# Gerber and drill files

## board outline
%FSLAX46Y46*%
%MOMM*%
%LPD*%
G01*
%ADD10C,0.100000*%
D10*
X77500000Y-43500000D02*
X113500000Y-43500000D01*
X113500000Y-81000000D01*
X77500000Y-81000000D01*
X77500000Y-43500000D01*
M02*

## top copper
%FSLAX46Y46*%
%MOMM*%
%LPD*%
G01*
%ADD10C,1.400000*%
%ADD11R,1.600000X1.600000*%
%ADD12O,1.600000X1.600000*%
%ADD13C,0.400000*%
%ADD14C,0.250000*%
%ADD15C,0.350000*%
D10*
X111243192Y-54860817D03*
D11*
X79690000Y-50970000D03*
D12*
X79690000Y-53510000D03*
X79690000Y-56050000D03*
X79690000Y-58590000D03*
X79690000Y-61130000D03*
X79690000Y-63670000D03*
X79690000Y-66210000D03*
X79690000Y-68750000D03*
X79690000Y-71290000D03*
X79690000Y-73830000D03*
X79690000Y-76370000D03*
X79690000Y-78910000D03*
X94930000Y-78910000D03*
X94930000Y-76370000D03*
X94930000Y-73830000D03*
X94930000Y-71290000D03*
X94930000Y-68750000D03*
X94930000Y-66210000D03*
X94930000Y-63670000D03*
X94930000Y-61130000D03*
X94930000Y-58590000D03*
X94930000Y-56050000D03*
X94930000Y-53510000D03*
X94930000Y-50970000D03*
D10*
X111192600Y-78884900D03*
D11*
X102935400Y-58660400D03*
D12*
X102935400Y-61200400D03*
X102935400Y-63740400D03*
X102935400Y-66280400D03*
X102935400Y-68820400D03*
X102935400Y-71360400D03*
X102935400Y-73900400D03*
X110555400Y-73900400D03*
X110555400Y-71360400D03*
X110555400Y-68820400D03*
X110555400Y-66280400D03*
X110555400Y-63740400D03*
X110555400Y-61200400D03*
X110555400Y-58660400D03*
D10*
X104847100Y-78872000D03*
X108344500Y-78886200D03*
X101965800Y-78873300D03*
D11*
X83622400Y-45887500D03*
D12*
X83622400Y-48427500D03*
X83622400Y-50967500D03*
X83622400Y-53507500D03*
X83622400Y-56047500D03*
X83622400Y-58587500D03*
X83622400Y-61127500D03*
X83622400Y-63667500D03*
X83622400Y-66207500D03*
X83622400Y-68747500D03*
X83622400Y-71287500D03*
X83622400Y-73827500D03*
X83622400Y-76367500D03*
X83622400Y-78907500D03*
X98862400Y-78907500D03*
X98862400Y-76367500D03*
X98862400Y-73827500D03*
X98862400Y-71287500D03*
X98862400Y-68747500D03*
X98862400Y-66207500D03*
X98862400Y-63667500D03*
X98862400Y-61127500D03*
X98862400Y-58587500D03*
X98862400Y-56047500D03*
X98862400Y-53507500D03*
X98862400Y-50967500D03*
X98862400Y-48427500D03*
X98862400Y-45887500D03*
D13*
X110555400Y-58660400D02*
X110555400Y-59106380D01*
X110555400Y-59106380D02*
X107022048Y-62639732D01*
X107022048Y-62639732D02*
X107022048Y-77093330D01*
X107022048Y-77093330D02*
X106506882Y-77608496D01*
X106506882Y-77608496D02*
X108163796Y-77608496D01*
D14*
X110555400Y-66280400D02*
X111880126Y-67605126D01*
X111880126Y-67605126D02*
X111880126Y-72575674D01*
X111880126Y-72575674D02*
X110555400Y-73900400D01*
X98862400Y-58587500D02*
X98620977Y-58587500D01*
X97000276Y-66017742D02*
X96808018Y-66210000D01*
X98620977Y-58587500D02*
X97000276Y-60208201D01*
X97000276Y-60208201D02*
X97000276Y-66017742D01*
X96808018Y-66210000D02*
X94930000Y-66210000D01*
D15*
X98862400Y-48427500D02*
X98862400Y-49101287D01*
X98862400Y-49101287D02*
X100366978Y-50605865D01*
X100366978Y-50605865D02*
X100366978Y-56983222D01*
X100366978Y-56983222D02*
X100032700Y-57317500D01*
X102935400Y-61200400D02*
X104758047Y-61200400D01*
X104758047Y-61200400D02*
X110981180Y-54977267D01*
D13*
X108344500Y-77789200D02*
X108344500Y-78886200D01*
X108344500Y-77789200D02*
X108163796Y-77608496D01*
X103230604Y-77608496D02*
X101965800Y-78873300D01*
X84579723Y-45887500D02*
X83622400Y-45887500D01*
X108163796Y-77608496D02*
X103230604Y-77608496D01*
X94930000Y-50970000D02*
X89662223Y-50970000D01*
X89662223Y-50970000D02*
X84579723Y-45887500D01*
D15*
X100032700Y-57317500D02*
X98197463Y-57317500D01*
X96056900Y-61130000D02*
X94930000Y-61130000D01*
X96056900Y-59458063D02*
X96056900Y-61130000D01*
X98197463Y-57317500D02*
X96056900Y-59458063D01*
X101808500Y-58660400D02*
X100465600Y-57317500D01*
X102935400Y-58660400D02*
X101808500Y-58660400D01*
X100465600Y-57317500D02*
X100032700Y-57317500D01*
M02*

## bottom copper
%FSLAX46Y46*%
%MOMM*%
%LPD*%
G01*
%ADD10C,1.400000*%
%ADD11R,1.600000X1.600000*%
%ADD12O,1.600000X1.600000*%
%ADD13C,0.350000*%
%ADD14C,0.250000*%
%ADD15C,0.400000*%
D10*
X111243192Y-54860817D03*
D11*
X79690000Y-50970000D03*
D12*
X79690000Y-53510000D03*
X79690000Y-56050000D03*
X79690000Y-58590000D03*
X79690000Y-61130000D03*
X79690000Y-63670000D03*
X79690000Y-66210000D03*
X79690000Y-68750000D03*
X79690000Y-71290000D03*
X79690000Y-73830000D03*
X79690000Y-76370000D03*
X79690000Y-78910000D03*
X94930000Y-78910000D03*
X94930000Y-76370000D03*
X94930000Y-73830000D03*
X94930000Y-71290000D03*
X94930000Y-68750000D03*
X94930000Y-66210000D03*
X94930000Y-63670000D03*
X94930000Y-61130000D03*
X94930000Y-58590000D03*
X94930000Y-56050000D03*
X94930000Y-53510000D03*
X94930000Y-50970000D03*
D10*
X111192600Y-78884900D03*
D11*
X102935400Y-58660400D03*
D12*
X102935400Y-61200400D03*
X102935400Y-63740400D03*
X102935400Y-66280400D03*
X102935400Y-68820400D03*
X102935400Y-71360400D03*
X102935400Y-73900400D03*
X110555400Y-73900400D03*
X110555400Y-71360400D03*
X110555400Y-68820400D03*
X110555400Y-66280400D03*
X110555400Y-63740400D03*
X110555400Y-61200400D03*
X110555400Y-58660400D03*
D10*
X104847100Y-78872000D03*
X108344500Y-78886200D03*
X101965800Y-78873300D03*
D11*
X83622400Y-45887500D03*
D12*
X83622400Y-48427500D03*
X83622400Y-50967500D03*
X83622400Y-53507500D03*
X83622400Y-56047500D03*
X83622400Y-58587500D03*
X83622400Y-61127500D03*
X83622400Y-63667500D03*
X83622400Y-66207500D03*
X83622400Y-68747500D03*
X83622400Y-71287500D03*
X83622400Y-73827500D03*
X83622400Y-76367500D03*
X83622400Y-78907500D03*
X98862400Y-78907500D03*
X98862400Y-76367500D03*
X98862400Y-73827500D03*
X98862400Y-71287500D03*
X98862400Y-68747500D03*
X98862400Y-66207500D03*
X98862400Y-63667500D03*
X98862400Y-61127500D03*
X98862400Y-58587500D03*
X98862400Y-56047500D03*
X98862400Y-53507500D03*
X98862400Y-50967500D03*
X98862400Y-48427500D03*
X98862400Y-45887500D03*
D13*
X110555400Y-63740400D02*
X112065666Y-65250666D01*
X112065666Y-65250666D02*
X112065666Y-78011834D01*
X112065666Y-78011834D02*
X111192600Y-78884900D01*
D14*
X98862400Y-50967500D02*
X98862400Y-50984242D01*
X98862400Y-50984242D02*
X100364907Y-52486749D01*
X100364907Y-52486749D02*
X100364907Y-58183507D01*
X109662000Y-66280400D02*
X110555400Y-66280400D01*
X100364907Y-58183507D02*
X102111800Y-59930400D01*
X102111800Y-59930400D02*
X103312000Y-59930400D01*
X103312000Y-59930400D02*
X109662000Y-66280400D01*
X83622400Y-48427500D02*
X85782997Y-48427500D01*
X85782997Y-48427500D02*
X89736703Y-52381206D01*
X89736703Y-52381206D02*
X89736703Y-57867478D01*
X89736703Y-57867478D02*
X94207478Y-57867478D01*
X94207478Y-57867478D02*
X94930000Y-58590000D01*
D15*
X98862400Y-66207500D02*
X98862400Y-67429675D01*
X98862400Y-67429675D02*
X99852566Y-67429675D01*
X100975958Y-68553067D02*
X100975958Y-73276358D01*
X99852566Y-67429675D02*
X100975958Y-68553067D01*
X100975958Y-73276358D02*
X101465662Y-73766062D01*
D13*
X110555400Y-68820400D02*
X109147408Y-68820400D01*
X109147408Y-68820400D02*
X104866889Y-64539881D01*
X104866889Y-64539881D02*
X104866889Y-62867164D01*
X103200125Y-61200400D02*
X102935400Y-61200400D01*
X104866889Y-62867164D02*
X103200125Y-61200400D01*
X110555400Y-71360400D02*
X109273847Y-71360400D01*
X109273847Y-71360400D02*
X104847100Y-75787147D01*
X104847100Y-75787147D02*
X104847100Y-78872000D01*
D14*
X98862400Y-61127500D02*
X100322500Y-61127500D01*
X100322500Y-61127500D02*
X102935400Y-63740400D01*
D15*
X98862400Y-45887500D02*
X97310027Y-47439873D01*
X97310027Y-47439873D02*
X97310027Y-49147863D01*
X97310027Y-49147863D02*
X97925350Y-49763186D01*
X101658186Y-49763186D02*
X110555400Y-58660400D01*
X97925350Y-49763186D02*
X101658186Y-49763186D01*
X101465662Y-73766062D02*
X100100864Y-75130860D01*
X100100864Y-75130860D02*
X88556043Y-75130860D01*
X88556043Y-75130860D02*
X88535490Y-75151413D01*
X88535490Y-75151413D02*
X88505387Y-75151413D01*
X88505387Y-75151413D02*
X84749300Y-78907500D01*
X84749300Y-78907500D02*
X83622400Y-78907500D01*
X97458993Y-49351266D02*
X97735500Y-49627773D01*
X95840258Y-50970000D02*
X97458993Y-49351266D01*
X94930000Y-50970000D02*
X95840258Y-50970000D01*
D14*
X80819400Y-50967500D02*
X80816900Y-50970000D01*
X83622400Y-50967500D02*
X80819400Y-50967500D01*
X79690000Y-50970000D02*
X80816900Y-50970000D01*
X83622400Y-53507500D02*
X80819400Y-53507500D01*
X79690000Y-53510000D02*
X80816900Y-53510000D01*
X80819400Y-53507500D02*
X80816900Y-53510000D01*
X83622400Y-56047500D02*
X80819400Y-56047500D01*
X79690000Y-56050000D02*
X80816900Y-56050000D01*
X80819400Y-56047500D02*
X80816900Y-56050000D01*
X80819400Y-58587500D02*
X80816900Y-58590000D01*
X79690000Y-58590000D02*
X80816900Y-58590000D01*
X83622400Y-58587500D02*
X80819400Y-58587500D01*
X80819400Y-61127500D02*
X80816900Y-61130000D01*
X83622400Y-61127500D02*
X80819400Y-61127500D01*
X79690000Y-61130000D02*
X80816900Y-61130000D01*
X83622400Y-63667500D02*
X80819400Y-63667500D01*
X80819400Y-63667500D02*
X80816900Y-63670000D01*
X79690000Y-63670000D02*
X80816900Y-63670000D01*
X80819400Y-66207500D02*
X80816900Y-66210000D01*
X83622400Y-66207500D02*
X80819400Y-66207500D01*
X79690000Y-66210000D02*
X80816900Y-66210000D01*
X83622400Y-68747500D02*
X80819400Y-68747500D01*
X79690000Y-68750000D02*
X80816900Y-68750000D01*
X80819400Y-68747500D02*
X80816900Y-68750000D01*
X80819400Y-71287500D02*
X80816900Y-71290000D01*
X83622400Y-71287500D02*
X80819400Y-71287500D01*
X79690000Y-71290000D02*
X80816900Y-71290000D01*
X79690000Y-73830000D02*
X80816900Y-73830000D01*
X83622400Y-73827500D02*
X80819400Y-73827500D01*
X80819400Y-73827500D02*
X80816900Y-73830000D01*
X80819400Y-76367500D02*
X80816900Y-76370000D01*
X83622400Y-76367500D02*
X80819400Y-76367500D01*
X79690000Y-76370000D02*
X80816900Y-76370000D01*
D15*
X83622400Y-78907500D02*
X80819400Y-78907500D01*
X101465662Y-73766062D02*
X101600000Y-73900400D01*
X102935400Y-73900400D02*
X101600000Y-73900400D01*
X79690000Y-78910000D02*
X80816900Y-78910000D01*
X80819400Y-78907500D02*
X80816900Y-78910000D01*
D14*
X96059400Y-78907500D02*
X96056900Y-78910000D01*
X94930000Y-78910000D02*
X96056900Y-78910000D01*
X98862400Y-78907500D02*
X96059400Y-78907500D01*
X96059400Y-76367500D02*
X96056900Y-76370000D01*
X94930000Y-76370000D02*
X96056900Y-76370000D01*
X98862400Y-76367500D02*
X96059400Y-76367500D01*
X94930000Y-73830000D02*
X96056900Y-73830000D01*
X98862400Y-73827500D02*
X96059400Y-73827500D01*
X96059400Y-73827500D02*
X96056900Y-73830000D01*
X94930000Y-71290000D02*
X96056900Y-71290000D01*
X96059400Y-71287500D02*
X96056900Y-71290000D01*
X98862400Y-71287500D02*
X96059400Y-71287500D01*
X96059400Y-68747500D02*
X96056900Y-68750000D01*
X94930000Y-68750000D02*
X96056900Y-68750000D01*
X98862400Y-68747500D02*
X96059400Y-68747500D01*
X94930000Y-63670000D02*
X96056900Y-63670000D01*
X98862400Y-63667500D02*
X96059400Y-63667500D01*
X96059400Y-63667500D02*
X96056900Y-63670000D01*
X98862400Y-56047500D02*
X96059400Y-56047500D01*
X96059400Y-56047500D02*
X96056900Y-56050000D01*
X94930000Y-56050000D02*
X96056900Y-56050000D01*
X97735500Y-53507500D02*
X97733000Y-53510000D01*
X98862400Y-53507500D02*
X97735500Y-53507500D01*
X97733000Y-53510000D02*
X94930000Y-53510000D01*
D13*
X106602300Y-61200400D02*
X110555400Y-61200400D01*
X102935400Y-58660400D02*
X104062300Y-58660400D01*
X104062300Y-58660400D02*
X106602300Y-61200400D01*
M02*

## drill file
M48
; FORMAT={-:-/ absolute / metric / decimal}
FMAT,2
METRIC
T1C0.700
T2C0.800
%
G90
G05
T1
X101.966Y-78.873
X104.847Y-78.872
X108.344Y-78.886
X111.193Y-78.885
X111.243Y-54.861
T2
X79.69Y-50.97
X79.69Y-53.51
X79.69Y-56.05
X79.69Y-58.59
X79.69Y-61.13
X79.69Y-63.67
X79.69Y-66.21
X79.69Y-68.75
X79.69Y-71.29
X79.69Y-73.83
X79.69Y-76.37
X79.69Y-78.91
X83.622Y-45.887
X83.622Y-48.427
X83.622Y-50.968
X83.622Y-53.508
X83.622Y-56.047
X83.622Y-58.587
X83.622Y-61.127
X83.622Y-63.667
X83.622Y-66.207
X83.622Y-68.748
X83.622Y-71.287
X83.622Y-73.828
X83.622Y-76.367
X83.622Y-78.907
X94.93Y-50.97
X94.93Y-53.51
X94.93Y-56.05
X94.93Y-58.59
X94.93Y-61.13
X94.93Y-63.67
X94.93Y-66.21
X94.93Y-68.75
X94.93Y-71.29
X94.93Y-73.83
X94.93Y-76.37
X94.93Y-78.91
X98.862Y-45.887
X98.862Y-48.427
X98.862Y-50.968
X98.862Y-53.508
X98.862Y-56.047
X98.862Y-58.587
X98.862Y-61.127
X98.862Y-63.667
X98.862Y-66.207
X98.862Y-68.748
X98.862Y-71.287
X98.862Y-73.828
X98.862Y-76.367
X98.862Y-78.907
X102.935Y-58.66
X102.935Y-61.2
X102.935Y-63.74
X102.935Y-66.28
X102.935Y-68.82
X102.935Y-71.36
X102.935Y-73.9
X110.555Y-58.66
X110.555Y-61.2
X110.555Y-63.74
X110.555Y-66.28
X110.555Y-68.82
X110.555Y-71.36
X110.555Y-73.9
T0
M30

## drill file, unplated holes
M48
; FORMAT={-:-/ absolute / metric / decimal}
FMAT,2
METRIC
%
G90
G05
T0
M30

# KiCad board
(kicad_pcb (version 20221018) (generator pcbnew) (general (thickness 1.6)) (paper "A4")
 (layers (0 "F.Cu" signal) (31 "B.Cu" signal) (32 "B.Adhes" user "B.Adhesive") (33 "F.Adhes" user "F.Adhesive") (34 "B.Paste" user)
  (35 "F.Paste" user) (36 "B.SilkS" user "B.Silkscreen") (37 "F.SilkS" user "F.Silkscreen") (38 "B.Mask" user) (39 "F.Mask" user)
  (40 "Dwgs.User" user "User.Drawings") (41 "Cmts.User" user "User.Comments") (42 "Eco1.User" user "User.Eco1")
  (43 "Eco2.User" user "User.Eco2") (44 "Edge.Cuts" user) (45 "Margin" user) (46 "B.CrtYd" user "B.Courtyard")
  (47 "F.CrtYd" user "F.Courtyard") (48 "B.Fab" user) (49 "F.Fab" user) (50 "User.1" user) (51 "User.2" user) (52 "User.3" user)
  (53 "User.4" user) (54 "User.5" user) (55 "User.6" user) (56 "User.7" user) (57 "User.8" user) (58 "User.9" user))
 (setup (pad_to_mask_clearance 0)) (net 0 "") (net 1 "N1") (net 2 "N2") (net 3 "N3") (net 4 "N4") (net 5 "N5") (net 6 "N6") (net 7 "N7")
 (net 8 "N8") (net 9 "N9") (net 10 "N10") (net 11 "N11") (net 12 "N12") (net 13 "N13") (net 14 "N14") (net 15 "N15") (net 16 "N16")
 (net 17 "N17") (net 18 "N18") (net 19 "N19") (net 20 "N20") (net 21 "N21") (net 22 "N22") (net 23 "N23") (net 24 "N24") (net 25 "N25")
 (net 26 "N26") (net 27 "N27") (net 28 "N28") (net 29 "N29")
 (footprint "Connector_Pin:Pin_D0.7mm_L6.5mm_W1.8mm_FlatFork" (layer "F.Cu") (at 111.243192 54.860817)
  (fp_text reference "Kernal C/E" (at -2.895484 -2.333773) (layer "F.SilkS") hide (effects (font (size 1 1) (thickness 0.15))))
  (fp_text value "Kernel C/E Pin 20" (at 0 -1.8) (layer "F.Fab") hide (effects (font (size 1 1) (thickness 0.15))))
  (pad "1" thru_hole circle (at 0 0) (size 1.4 1.4) (drill 0.7) (layers "*.Cu" "*.Mask") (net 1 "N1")))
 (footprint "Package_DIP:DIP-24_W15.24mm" (layer "F.Cu") (at 79.69 50.97)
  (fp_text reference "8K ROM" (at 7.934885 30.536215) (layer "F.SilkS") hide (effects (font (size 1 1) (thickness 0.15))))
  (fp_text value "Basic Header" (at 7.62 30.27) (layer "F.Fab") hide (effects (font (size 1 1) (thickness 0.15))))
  (pad "1" thru_hole rect (at 0 0) (size 1.6 1.6) (drill 0.8) (layers "*.Cu" "*.Mask") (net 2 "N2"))
  (pad "2" thru_hole oval (at 0 2.54) (size 1.6 1.6) (drill 0.8) (layers "*.Cu" "*.Mask") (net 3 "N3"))
  (pad "3" thru_hole oval (at 0 5.08) (size 1.6 1.6) (drill 0.8) (layers "*.Cu" "*.Mask") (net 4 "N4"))
  (pad "4" thru_hole oval (at 0 7.62) (size 1.6 1.6) (drill 0.8) (layers "*.Cu" "*.Mask") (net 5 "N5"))
  (pad "5" thru_hole oval (at 0 10.16) (size 1.6 1.6) (drill 0.8) (layers "*.Cu" "*.Mask") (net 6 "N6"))
  (pad "6" thru_hole oval (at 0 12.7) (size 1.6 1.6) (drill 0.8) (layers "*.Cu" "*.Mask") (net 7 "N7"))
  (pad "7" thru_hole oval (at 0 15.24) (size 1.6 1.6) (drill 0.8) (layers "*.Cu" "*.Mask") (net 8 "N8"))
  (pad "8" thru_hole oval (at 0 17.78) (size 1.6 1.6) (drill 0.8) (layers "*.Cu" "*.Mask") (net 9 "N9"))
  (pad "9" thru_hole oval (at 0 20.32) (size 1.6 1.6) (drill 0.8) (layers "*.Cu" "*.Mask") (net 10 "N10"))
  (pad "10" thru_hole oval (at 0 22.86) (size 1.6 1.6) (drill 0.8) (layers "*.Cu" "*.Mask") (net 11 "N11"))
  (pad "11" thru_hole oval (at 0 25.4) (size 1.6 1.6) (drill 0.8) (layers "*.Cu" "*.Mask") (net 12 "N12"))
  (pad "12" thru_hole oval (at 0 27.94) (size 1.6 1.6) (drill 0.8) (layers "*.Cu" "*.Mask") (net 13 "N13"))
  (pad "13" thru_hole oval (at 15.24 27.94) (size 1.6 1.6) (drill 0.8) (layers "*.Cu" "*.Mask") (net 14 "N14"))
  (pad "14" thru_hole oval (at 15.24 25.4) (size 1.6 1.6) (drill 0.8) (layers "*.Cu" "*.Mask") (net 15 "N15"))
  (pad "15" thru_hole oval (at 15.24 22.86) (size 1.6 1.6) (drill 0.8) (layers "*.Cu" "*.Mask") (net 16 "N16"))
  (pad "16" thru_hole oval (at 15.24 20.32) (size 1.6 1.6) (drill 0.8) (layers "*.Cu" "*.Mask") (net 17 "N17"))
  (pad "17" thru_hole oval (at 15.24 17.78) (size 1.6 1.6) (drill 0.8) (layers "*.Cu" "*.Mask") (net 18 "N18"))
  (pad "18" thru_hole oval (at 15.24 15.24) (size 1.6 1.6) (drill 0.8) (layers "*.Cu" "*.Mask") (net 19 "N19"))
  (pad "19" thru_hole oval (at 15.24 12.7) (size 1.6 1.6) (drill 0.8) (layers "*.Cu" "*.Mask") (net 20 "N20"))
  (pad "20" thru_hole oval (at 15.24 10.16) (size 1.6 1.6) (drill 0.8) (layers "*.Cu" "*.Mask") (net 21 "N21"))
  (pad "21" thru_hole oval (at 15.24 7.62) (size 1.6 1.6) (drill 0.8) (layers "*.Cu" "*.Mask") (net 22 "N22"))
  (pad "22" thru_hole oval (at 15.24 5.08) (size 1.6 1.6) (drill 0.8) (layers "*.Cu" "*.Mask") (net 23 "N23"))
  (pad "23" thru_hole oval (at 15.24 2.54) (size 1.6 1.6) (drill 0.8) (layers "*.Cu" "*.Mask") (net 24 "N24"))
  (pad "24" thru_hole oval (at 15.24 0) (size 1.6 1.6) (drill 0.8) (layers "*.Cu" "*.Mask") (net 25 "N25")))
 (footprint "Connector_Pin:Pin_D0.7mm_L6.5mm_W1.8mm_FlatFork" (layer "F.Cu") (at 111.1926 78.8849)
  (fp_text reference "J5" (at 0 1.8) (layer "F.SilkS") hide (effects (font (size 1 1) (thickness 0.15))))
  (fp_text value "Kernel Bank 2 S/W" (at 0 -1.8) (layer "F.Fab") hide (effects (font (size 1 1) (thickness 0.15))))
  (pad "1" thru_hole circle (at 0 0) (size 1.4 1.4) (drill 0.7) (layers "*.Cu" "*.Mask") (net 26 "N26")))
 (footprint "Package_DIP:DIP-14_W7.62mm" (layer "F.Cu") (at 102.9354 58.6604)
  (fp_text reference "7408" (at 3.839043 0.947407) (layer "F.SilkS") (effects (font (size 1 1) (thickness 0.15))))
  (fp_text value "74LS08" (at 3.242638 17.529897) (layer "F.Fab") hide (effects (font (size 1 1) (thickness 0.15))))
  (pad "1" thru_hole rect (at 0 0) (size 1.6 1.6) (drill 0.8) (layers "*.Cu" "*.Mask") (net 21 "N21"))
  (pad "2" thru_hole oval (at 0 2.54) (size 1.6 1.6) (drill 0.8) (layers "*.Cu" "*.Mask") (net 1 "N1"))
  (pad "3" thru_hole oval (at 0 5.08) (size 1.6 1.6) (drill 0.8) (layers "*.Cu" "*.Mask") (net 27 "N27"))
  (pad "4" thru_hole oval (at 0 7.62) (size 1.6 1.6) (drill 0.8) (layers "*.Cu" "*.Mask"))
  (pad "5" thru_hole oval (at 0 10.16) (size 1.6 1.6) (drill 0.8) (layers "*.Cu" "*.Mask"))
  (pad "6" thru_hole oval (at 0 12.7) (size 1.6 1.6) (drill 0.8) (layers "*.Cu" "*.Mask"))
  (pad "7" thru_hole oval (at 0 15.24) (size 1.6 1.6) (drill 0.8) (layers "*.Cu" "*.Mask") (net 13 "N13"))
  (pad "8" thru_hole oval (at 7.62 15.24) (size 1.6 1.6) (drill 0.8) (layers "*.Cu" "*.Mask") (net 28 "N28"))
  (pad "9" thru_hole oval (at 7.62 12.7) (size 1.6 1.6) (drill 0.8) (layers "*.Cu" "*.Mask") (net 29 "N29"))
  (pad "10" thru_hole oval (at 7.62 10.16) (size 1.6 1.6) (drill 0.8) (layers "*.Cu" "*.Mask") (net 1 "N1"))
  (pad "11" thru_hole oval (at 7.62 7.62) (size 1.6 1.6) (drill 0.8) (layers "*.Cu" "*.Mask") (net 28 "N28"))
  (pad "12" thru_hole oval (at 7.62 5.08) (size 1.6 1.6) (drill 0.8) (layers "*.Cu" "*.Mask") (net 26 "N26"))
  (pad "13" thru_hole oval (at 7.62 2.54) (size 1.6 1.6) (drill 0.8) (layers "*.Cu" "*.Mask") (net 21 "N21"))
  (pad "14" thru_hole oval (at 7.62 0) (size 1.6 1.6) (drill 0.8) (layers "*.Cu" "*.Mask") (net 25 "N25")))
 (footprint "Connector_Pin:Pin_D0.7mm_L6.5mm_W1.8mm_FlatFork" (layer "F.Cu") (at 104.8471 78.872)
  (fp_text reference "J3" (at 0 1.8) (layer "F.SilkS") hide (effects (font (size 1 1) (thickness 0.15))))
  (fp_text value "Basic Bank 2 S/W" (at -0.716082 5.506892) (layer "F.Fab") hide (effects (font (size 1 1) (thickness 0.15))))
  (pad "1" thru_hole circle (at 0 0) (size 1.4 1.4) (drill 0.7) (layers "*.Cu" "*.Mask") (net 29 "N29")))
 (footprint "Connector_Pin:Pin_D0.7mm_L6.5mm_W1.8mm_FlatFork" (layer "F.Cu") (at 108.3445 78.8862)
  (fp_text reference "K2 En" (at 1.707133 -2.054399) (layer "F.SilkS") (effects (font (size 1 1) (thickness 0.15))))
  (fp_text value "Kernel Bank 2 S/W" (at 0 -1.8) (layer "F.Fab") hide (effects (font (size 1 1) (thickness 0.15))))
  (pad "1" thru_hole circle (at 0 0) (size 1.4 1.4) (drill 0.7) (layers "*.Cu" "*.Mask") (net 25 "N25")))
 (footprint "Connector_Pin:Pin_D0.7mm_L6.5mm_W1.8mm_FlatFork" (layer "F.Cu") (at 101.9658 78.8733)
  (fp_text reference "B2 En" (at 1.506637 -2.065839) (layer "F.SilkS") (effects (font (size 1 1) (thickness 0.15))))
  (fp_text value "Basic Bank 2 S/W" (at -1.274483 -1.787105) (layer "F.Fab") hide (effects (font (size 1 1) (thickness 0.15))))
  (pad "1" thru_hole circle (at 0 0) (size 1.4 1.4) (drill 0.7) (layers "*.Cu" "*.Mask") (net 25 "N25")))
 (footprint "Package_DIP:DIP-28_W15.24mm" (layer "F.Cu") (at 83.6224 45.8875)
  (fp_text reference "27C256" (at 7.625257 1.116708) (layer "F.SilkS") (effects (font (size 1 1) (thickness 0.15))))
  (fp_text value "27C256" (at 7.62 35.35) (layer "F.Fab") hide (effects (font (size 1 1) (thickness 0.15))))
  (pad "1" thru_hole rect (at 0 0) (size 1.6 1.6) (drill 0.8) (layers "*.Cu" "*.Mask") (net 25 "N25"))
  (pad "2" thru_hole oval (at 0 2.54) (size 1.6 1.6) (drill 0.8) (layers "*.Cu" "*.Mask") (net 22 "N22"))
  (pad "3" thru_hole oval (at 0 5.08) (size 1.6 1.6) (drill 0.8) (layers "*.Cu" "*.Mask") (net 2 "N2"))
  (pad "4" thru_hole oval (at 0 7.62) (size 1.6 1.6) (drill 0.8) (layers "*.Cu" "*.Mask") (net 3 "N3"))
  (pad "5" thru_hole oval (at 0 10.16) (size 1.6 1.6) (drill 0.8) (layers "*.Cu" "*.Mask") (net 4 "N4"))
  (pad "6" thru_hole oval (at 0 12.7) (size 1.6 1.6) (drill 0.8) (layers "*.Cu" "*.Mask") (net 5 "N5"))
  (pad "7" thru_hole oval (at 0 15.24) (size 1.6 1.6) (drill 0.8) (layers "*.Cu" "*.Mask") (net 6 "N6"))
  (pad "8" thru_hole oval (at 0 17.78) (size 1.6 1.6) (drill 0.8) (layers "*.Cu" "*.Mask") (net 7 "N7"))
  (pad "9" thru_hole oval (at 0 20.32) (size 1.6 1.6) (drill 0.8) (layers "*.Cu" "*.Mask") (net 8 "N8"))
  (pad "10" thru_hole oval (at 0 22.86) (size 1.6 1.6) (drill 0.8) (layers "*.Cu" "*.Mask") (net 9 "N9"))
  (pad "11" thru_hole oval (at 0 25.4) (size 1.6 1.6) (drill 0.8) (layers "*.Cu" "*.Mask") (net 10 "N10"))
  (pad "12" thru_hole oval (at 0 27.94) (size 1.6 1.6) (drill 0.8) (layers "*.Cu" "*.Mask") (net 11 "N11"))
  (pad "13" thru_hole oval (at 0 30.48) (size 1.6 1.6) (drill 0.8) (layers "*.Cu" "*.Mask") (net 12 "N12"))
  (pad "14" thru_hole oval (at 0 33.02) (size 1.6 1.6) (drill 0.8) (layers "*.Cu" "*.Mask") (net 13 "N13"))
  (pad "15" thru_hole oval (at 15.24 33.02) (size 1.6 1.6) (drill 0.8) (layers "*.Cu" "*.Mask") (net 14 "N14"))
  (pad "16" thru_hole oval (at 15.24 30.48) (size 1.6 1.6) (drill 0.8) (layers "*.Cu" "*.Mask") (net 15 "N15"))
  (pad "17" thru_hole oval (at 15.24 27.94) (size 1.6 1.6) (drill 0.8) (layers "*.Cu" "*.Mask") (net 16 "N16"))
  (pad "18" thru_hole oval (at 15.24 25.4) (size 1.6 1.6) (drill 0.8) (layers "*.Cu" "*.Mask") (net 17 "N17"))
  (pad "19" thru_hole oval (at 15.24 22.86) (size 1.6 1.6) (drill 0.8) (layers "*.Cu" "*.Mask") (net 18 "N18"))
  (pad "20" thru_hole oval (at 15.24 20.32) (size 1.6 1.6) (drill 0.8) (layers "*.Cu" "*.Mask") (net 13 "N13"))
  (pad "21" thru_hole oval (at 15.24 17.78) (size 1.6 1.6) (drill 0.8) (layers "*.Cu" "*.Mask") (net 20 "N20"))
  (pad "22" thru_hole oval (at 15.24 15.24) (size 1.6 1.6) (drill 0.8) (layers "*.Cu" "*.Mask") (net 27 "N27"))
  (pad "23" thru_hole oval (at 15.24 12.7) (size 1.6 1.6) (drill 0.8) (layers "*.Cu" "*.Mask") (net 19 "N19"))
  (pad "24" thru_hole oval (at 15.24 10.16) (size 1.6 1.6) (drill 0.8) (layers "*.Cu" "*.Mask") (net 23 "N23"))
  (pad "25" thru_hole oval (at 15.24 7.62) (size 1.6 1.6) (drill 0.8) (layers "*.Cu" "*.Mask") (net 24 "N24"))
  (pad "26" thru_hole oval (at 15.24 5.08) (size 1.6 1.6) (drill 0.8) (layers "*.Cu" "*.Mask") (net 28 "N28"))
  (pad "27" thru_hole oval (at 15.24 2.54) (size 1.6 1.6) (drill 0.8) (layers "*.Cu" "*.Mask") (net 21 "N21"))
  (pad "28" thru_hole oval (at 15.24 0) (size 1.6 1.6) (drill 0.8) (layers "*.Cu" "*.Mask") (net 25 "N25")))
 (gr_rect (start 77.5 43.5) (end 113.5 81) (stroke (width 0.1) (type default)) (fill none) (layer "Edge.Cuts"))
 (segment (start 102.9354 61.2004) (end 104.758047 61.2004) (width 0.35) (layer "F.Cu") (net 1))
 (segment (start 104.758047 61.2004) (end 110.98118 54.977267) (width 0.35) (layer "F.Cu") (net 1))
 (segment (start 109.147408 68.8204) (end 104.866889 64.539881) (width 0.35) (layer "B.Cu") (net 1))
 (segment (start 103.200125 61.2004) (end 102.9354 61.2004) (width 0.35) (layer "B.Cu") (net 1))
 (segment (start 104.866889 62.867164) (end 103.200125 61.2004) (width 0.35) (layer "B.Cu") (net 1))
 (segment (start 104.866889 64.539881) (end 104.866889 62.867164) (width 0.35) (layer "B.Cu") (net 1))
 (segment (start 110.5554 68.8204) (end 109.147408 68.8204) (width 0.35) (layer "B.Cu") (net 1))
 (segment (start 108.3445 77.7892) (end 108.3445 78.8862) (width 0.4) (layer "F.Cu") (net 25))
 (segment (start 108.3445 77.7892) (end 108.163796 77.608496) (width 0.4) (layer "F.Cu") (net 25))
 (segment (start 103.230604 77.608496) (end 101.9658 78.8733) (width 0.4) (layer "F.Cu") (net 25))
 (segment (start 84.579723 45.8875) (end 83.6224 45.8875) (width 0.4) (layer "F.Cu") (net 25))
 (segment (start 107.022048 62.639732) (end 107.022048 77.09333) (width 0.4) (layer "F.Cu") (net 25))
 (segment (start 110.5554 58.6604) (end 110.5554 59.10638) (width 0.4) (layer "F.Cu") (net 25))
 (segment (start 108.163796 77.608496) (end 103.230604 77.608496) (width 0.4) (layer "F.Cu") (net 25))
 (segment (start 110.5554 59.10638) (end 107.022048 62.639732) (width 0.4) (layer "F.Cu") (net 25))
 (segment (start 94.93 50.97) (end 89.662223 50.97) (width 0.4) (layer "F.Cu") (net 25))
 (segment (start 106.506882 77.608496) (end 108.163796 77.608496) (width 0.4) (layer "F.Cu") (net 25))
 (segment (start 89.662223 50.97) (end 84.579723 45.8875) (width 0.4) (layer "F.Cu") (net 25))
 (segment (start 107.022048 77.09333) (end 106.506882 77.608496) (width 0.4) (layer "F.Cu") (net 25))
 (segment (start 101.658186 49.763186) (end 110.5554 58.6604) (width 0.4) (layer "B.Cu") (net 25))
 (segment (start 97.92535 49.763186) (end 101.658186 49.763186) (width 0.4) (layer "B.Cu") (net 25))
 (segment (start 98.8624 45.8875) (end 97.310027 47.439873) (width 0.4) (layer "B.Cu") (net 25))
 (segment (start 97.310027 49.147863) (end 97.92535 49.763186) (width 0.4) (layer "B.Cu") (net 25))
 (segment (start 97.458993 49.351266) (end 97.7355 49.627773) (width 0.4) (layer "B.Cu") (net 25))
 (segment (start 97.310027 47.439873) (end 97.310027 49.147863) (width 0.4) (layer "B.Cu") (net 25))
 (segment (start 95.840258 50.97) (end 97.458993 49.351266) (width 0.4) (layer "B.Cu") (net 25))
 (segment (start 94.93 50.97) (end 95.840258 50.97) (width 0.4) (layer "B.Cu") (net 25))
 (segment (start 109.273847 71.3604) (end 104.8471 75.787147) (width 0.35) (layer "B.Cu") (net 29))
 (segment (start 110.5554 71.3604) (end 109.273847 71.3604) (width 0.35) (layer "B.Cu") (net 29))
 (segment (start 104.8471 75.787147) (end 104.8471 78.872) (width 0.35) (layer "B.Cu") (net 29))
 (segment (start 112.065666 78.011834) (end 111.1926 78.8849) (width 0.35) (layer "B.Cu") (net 26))
 (segment (start 112.065666 65.250666) (end 112.065666 78.011834) (width 0.35) (layer "B.Cu") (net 26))
 (segment (start 110.5554 63.7404) (end 112.065666 65.250666) (width 0.35) (layer "B.Cu") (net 26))
 (segment (start 89.736703 57.867478) (end 94.207478 57.867478) (width 0.25) (layer "B.Cu") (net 22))
 (segment (start 94.207478 57.867478) (end 94.93 58.59) (width 0.25) (layer "B.Cu") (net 22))
 (segment (start 83.6224 48.4275) (end 85.782997 48.4275) (width 0.25) (layer "B.Cu") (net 22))
 (segment (start 89.736703 52.381206) (end 89.736703 57.867478) (width 0.25) (layer "B.Cu") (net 22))
 (segment (start 85.782997 48.4275) (end 89.736703 52.381206) (width 0.25) (layer "B.Cu") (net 22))
 (segment (start 80.8194 50.9675) (end 80.8169 50.97) (width 0.25) (layer "B.Cu") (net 2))
 (segment (start 83.6224 50.9675) (end 80.8194 50.9675) (width 0.25) (layer "B.Cu") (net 2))
 (segment (start 79.69 50.97) (end 80.8169 50.97) (width 0.25) (layer "B.Cu") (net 2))
 (segment (start 83.6224 53.5075) (end 80.8194 53.5075) (width 0.25) (layer "B.Cu") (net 3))
 (segment (start 79.69 53.51) (end 80.8169 53.51) (width 0.25) (layer "B.Cu") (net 3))
 (segment (start 80.8194 53.5075) (end 80.8169 53.51) (width 0.25) (layer "B.Cu") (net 3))
 (segment (start 83.6224 56.0475) (end 80.8194 56.0475) (width 0.25) (layer "B.Cu") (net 4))
 (segment (start 79.69 56.05) (end 80.8169 56.05) (width 0.25) (layer "B.Cu") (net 4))
 (segment (start 80.8194 56.0475) (end 80.8169 56.05) (width 0.25) (layer "B.Cu") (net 4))
 (segment (start 80.8194 58.5875) (end 80.8169 58.59) (width 0.25) (layer "B.Cu") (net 5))
 (segment (start 79.69 58.59) (end 80.8169 58.59) (width 0.25) (layer "B.Cu") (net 5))
 (segment (start 83.6224 58.5875) (end 80.8194 58.5875) (width 0.25) (layer "B.Cu") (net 5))
 (segment (start 80.8194 61.1275) (end 80.8169 61.13) (width 0.25) (layer "B.Cu") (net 6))
 (segment (start 83.6224 61.1275) (end 80.8194 61.1275) (width 0.25) (layer "B.Cu") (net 6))
 (segment (start 79.69 61.13) (end 80.8169 61.13) (width 0.25) (layer "B.Cu") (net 6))
 (segment (start 83.6224 63.6675) (end 80.8194 63.6675) (width 0.25) (layer "B.Cu") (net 7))
 (segment (start 80.8194 63.6675) (end 80.8169 63.67) (width 0.25) (layer "B.Cu") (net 7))
 (segment (start 79.69 63.67) (end 80.8169 63.67) (width 0.25) (layer "B.Cu") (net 7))
 (segment (start 80.8194 66.2075) (end 80.8169 66.21) (width 0.25) (layer "B.Cu") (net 8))
 (segment (start 83.6224 66.2075) (end 80.8194 66.2075) (width 0.25) (layer "B.Cu") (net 8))
 (segment (start 79.69 66.21) (end 80.8169 66.21) (width 0.25) (layer "B.Cu") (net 8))
 (segment (start 83.6224 68.7475) (end 80.8194 68.7475) (width 0.25) (layer "B.Cu") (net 9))
 (segment (start 79.69 68.75) (end 80.8169 68.75) (width 0.25) (layer "B.Cu") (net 9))
 (segment (start 80.8194 68.7475) (end 80.8169 68.75) (width 0.25) (layer "B.Cu") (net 9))
 (segment (start 80.8194 71.2875) (end 80.8169 71.29) (width 0.25) (layer "B.Cu") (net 10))
 (segment (start 83.6224 71.2875) (end 80.8194 71.2875) (width 0.25) (layer "B.Cu") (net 10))
 (segment (start 79.69 71.29) (end 80.8169 71.29) (width 0.25) (layer "B.Cu") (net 10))
 (segment (start 79.69 73.83) (end 80.8169 73.83) (width 0.25) (layer "B.Cu") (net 11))
 (segment (start 83.6224 73.8275) (end 80.8194 73.8275) (width 0.25) (layer "B.Cu") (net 11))
 (segment (start 80.8194 73.8275) (end 80.8169 73.83) (width 0.25) (layer "B.Cu") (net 11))
 (segment (start 80.8194 76.3675) (end 80.8169 76.37) (width 0.25) (layer "B.Cu") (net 12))
 (segment (start 83.6224 76.3675) (end 80.8194 76.3675) (width 0.25) (layer "B.Cu") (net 12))
 (segment (start 79.69 76.37) (end 80.8169 76.37) (width 0.25) (layer "B.Cu") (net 12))
 (segment (start 83.6224 78.9075) (end 80.8194 78.9075) (width 0.4) (layer "B.Cu") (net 13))
 (segment (start 88.556043 75.13086) (end 88.53549 75.151413) (width 0.4) (layer "B.Cu") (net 13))
 (segment (start 88.53549 75.151413) (end 88.505387 75.151413) (width 0.4) (layer "B.Cu") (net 13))
 (segment (start 98.8624 66.2075) (end 98.8624 67.429675) (width 0.4) (layer "B.Cu") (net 13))
 (segment (start 100.975958 68.553067) (end 100.975958 73.276358) (width 0.4) (layer "B.Cu") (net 13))
 (segment (start 100.975958 73.276358) (end 101.465662 73.766062) (width 0.4) (layer "B.Cu") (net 13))
 (segment (start 101.465662 73.766062) (end 101.6 73.9004) (width 0.4) (layer "B.Cu") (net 13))
 (segment (start 99.852566 67.429675) (end 100.975958 68.553067) (width 0.4) (layer "B.Cu") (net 13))
 (segment (start 101.465662 73.766062) (end 100.100864 75.13086) (width 0.4) (layer "B.Cu") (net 13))
 (segment (start 102.9354 73.9004) (end 101.6 73.9004) (width 0.4) (layer "B.Cu") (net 13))
 (segment (start 100.100864 75.13086) (end 88.556043 75.13086) (width 0.4) (layer "B.Cu") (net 13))
 (segment (start 79.69 78.91) (end 80.8169 78.91) (width 0.4) (layer "B.Cu") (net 13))
 (segment (start 98.8624 67.429675) (end 99.852566 67.429675) (width 0.4) (layer "B.Cu") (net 13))
 (segment (start 84.7493 78.9075) (end 83.6224 78.9075) (width 0.4) (layer "B.Cu") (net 13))
 (segment (start 80.8194 78.9075) (end 80.8169 78.91) (width 0.4) (layer "B.Cu") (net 13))
 (segment (start 88.505387 75.151413) (end 84.7493 78.9075) (width 0.4) (layer "B.Cu") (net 13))
 (segment (start 96.0594 78.9075) (end 96.0569 78.91) (width 0.25) (layer "B.Cu") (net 14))
 (segment (start 94.93 78.91) (end 96.0569 78.91) (width 0.25) (layer "B.Cu") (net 14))
 (segment (start 98.8624 78.9075) (end 96.0594 78.9075) (width 0.25) (layer "B.Cu") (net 14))
 (segment (start 96.0594 76.3675) (end 96.0569 76.37) (width 0.25) (layer "B.Cu") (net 15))
 (segment (start 94.93 76.37) (end 96.0569 76.37) (width 0.25) (layer "B.Cu") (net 15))
 (segment (start 98.8624 76.3675) (end 96.0594 76.3675) (width 0.25) (layer "B.Cu") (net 15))
 (segment (start 94.93 73.83) (end 96.0569 73.83) (width 0.25) (layer "B.Cu") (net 16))
 (segment (start 98.8624 73.8275) (end 96.0594 73.8275) (width 0.25) (layer "B.Cu") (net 16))
 (segment (start 96.0594 73.8275) (end 96.0569 73.83) (width 0.25) (layer "B.Cu") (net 16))
 (segment (start 94.93 71.29) (end 96.0569 71.29) (width 0.25) (layer "B.Cu") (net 17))
 (segment (start 96.0594 71.2875) (end 96.0569 71.29) (width 0.25) (layer "B.Cu") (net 17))
 (segment (start 98.8624 71.2875) (end 96.0594 71.2875) (width 0.25) (layer "B.Cu") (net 17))
 (segment (start 96.0594 68.7475) (end 96.0569 68.75) (width 0.25) (layer "B.Cu") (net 18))
 (segment (start 94.93 68.75) (end 96.0569 68.75) (width 0.25) (layer "B.Cu") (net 18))
 (segment (start 98.8624 68.7475) (end 96.0594 68.7475) (width 0.25) (layer "B.Cu") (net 18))
 (segment (start 94.93 63.67) (end 96.0569 63.67) (width 0.25) (layer "B.Cu") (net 20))
 (segment (start 98.8624 63.6675) (end 96.0594 63.6675) (width 0.25) (layer "B.Cu") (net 20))
 (segment (start 96.0594 63.6675) (end 96.0569 63.67) (width 0.25) (layer "B.Cu") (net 20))
 (segment (start 98.8624 61.1275) (end 100.3225 61.1275) (width 0.25) (layer "B.Cu") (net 27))
 (segment (start 100.3225 61.1275) (end 102.9354 63.7404) (width 0.25) (layer "B.Cu") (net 27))
 (segment (start 97.000276 66.017742) (end 96.808018 66.21) (width 0.25) (layer "F.Cu") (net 19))
 (segment (start 97.000276 60.208201) (end 97.000276 66.017742) (width 0.25) (layer "F.Cu") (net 19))
 (segment (start 98.8624 58.5875) (end 98.620977 58.5875) (width 0.25) (layer "F.Cu") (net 19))
 (segment (start 96.808018 66.21) (end 94.93 66.21) (width 0.25) (layer "F.Cu") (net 19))
 (segment (start 98.620977 58.5875) (end 97.000276 60.208201) (width 0.25) (layer "F.Cu") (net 19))
 (segment (start 98.8624 56.0475) (end 96.0594 56.0475) (width 0.25) (layer "B.Cu") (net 23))
 (segment (start 96.0594 56.0475) (end 96.0569 56.05) (width 0.25) (layer "B.Cu") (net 23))
 (segment (start 94.93 56.05) (end 96.0569 56.05) (width 0.25) (layer "B.Cu") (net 23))
 (segment (start 97.7355 53.5075) (end 97.733 53.51) (width 0.25) (layer "B.Cu") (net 24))
 (segment (start 98.8624 53.5075) (end 97.7355 53.5075) (width 0.25) (layer "B.Cu") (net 24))
 (segment (start 97.733 53.51) (end 94.93 53.51) (width 0.25) (layer "B.Cu") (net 24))
 (segment (start 111.880126 72.575674) (end 110.5554 73.9004) (width 0.25) (layer "F.Cu") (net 28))
 (segment (start 111.880126 67.605126) (end 111.880126 72.575674) (width 0.25) (layer "F.Cu") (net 28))
 (segment (start 110.5554 66.2804) (end 111.880126 67.605126) (width 0.25) (layer "F.Cu") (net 28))
 (segment (start 100.364907 58.183507) (end 102.1118 59.9304) (width 0.25) (layer "B.Cu") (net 28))
 (segment (start 98.8624 50.9675) (end 98.8624 50.984242) (width 0.25) (layer "B.Cu") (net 28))
 (segment (start 98.8624 50.984242) (end 100.364907 52.486749) (width 0.25) (layer "B.Cu") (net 28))
 (segment (start 102.1118 59.9304) (end 103.312 59.9304) (width 0.25) (layer "B.Cu") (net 28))
 (segment (start 109.662 66.2804) (end 110.5554 66.2804) (width 0.25) (layer "B.Cu") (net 28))
 (segment (start 100.364907 52.486749) (end 100.364907 58.183507) (width 0.25) (layer "B.Cu") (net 28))
 (segment (start 103.312 59.9304) (end 109.662 66.2804) (width 0.25) (layer "B.Cu") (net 28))
 (segment (start 100.0327 57.3175) (end 98.197463 57.3175) (width 0.35) (layer "F.Cu") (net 21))
 (segment (start 96.0569 61.13) (end 94.93 61.13) (width 0.35) (layer "F.Cu") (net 21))
 (segment (start 100.366978 56.983222) (end 100.0327 57.3175) (width 0.35) (layer "F.Cu") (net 21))
 (segment (start 96.0569 59.458063) (end 96.0569 61.13) (width 0.35) (layer "F.Cu") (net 21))
 (segment (start 98.197463 57.3175) (end 96.0569 59.458063) (width 0.35) (layer "F.Cu") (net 21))
 (segment (start 98.8624 49.101287) (end 100.366978 50.605865) (width 0.35) (layer "F.Cu") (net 21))
 (segment (start 98.8624 48.4275) (end 98.8624 49.101287) (width 0.35) (layer "F.Cu") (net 21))
 (segment (start 100.366978 50.605865) (end 100.366978 56.983222) (width 0.35) (layer "F.Cu") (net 21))
 (segment (start 101.8085 58.6604) (end 100.4656 57.3175) (width 0.35) (layer "F.Cu") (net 21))
 (segment (start 102.9354 58.6604) (end 101.8085 58.6604) (width 0.35) (layer "F.Cu") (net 21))
 (segment (start 100.4656 57.3175) (end 100.0327 57.3175) (width 0.35) (layer "F.Cu") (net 21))
 (segment (start 106.6023 61.2004) (end 110.5554 61.2004) (width 0.35) (layer "B.Cu") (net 21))
 (segment (start 102.9354 58.6604) (end 104.0623 58.6604) (width 0.35) (layer "B.Cu") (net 21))
 (segment (start 104.0623 58.6604) (end 106.6023 61.2004) (width 0.35) (layer "B.Cu") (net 21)))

